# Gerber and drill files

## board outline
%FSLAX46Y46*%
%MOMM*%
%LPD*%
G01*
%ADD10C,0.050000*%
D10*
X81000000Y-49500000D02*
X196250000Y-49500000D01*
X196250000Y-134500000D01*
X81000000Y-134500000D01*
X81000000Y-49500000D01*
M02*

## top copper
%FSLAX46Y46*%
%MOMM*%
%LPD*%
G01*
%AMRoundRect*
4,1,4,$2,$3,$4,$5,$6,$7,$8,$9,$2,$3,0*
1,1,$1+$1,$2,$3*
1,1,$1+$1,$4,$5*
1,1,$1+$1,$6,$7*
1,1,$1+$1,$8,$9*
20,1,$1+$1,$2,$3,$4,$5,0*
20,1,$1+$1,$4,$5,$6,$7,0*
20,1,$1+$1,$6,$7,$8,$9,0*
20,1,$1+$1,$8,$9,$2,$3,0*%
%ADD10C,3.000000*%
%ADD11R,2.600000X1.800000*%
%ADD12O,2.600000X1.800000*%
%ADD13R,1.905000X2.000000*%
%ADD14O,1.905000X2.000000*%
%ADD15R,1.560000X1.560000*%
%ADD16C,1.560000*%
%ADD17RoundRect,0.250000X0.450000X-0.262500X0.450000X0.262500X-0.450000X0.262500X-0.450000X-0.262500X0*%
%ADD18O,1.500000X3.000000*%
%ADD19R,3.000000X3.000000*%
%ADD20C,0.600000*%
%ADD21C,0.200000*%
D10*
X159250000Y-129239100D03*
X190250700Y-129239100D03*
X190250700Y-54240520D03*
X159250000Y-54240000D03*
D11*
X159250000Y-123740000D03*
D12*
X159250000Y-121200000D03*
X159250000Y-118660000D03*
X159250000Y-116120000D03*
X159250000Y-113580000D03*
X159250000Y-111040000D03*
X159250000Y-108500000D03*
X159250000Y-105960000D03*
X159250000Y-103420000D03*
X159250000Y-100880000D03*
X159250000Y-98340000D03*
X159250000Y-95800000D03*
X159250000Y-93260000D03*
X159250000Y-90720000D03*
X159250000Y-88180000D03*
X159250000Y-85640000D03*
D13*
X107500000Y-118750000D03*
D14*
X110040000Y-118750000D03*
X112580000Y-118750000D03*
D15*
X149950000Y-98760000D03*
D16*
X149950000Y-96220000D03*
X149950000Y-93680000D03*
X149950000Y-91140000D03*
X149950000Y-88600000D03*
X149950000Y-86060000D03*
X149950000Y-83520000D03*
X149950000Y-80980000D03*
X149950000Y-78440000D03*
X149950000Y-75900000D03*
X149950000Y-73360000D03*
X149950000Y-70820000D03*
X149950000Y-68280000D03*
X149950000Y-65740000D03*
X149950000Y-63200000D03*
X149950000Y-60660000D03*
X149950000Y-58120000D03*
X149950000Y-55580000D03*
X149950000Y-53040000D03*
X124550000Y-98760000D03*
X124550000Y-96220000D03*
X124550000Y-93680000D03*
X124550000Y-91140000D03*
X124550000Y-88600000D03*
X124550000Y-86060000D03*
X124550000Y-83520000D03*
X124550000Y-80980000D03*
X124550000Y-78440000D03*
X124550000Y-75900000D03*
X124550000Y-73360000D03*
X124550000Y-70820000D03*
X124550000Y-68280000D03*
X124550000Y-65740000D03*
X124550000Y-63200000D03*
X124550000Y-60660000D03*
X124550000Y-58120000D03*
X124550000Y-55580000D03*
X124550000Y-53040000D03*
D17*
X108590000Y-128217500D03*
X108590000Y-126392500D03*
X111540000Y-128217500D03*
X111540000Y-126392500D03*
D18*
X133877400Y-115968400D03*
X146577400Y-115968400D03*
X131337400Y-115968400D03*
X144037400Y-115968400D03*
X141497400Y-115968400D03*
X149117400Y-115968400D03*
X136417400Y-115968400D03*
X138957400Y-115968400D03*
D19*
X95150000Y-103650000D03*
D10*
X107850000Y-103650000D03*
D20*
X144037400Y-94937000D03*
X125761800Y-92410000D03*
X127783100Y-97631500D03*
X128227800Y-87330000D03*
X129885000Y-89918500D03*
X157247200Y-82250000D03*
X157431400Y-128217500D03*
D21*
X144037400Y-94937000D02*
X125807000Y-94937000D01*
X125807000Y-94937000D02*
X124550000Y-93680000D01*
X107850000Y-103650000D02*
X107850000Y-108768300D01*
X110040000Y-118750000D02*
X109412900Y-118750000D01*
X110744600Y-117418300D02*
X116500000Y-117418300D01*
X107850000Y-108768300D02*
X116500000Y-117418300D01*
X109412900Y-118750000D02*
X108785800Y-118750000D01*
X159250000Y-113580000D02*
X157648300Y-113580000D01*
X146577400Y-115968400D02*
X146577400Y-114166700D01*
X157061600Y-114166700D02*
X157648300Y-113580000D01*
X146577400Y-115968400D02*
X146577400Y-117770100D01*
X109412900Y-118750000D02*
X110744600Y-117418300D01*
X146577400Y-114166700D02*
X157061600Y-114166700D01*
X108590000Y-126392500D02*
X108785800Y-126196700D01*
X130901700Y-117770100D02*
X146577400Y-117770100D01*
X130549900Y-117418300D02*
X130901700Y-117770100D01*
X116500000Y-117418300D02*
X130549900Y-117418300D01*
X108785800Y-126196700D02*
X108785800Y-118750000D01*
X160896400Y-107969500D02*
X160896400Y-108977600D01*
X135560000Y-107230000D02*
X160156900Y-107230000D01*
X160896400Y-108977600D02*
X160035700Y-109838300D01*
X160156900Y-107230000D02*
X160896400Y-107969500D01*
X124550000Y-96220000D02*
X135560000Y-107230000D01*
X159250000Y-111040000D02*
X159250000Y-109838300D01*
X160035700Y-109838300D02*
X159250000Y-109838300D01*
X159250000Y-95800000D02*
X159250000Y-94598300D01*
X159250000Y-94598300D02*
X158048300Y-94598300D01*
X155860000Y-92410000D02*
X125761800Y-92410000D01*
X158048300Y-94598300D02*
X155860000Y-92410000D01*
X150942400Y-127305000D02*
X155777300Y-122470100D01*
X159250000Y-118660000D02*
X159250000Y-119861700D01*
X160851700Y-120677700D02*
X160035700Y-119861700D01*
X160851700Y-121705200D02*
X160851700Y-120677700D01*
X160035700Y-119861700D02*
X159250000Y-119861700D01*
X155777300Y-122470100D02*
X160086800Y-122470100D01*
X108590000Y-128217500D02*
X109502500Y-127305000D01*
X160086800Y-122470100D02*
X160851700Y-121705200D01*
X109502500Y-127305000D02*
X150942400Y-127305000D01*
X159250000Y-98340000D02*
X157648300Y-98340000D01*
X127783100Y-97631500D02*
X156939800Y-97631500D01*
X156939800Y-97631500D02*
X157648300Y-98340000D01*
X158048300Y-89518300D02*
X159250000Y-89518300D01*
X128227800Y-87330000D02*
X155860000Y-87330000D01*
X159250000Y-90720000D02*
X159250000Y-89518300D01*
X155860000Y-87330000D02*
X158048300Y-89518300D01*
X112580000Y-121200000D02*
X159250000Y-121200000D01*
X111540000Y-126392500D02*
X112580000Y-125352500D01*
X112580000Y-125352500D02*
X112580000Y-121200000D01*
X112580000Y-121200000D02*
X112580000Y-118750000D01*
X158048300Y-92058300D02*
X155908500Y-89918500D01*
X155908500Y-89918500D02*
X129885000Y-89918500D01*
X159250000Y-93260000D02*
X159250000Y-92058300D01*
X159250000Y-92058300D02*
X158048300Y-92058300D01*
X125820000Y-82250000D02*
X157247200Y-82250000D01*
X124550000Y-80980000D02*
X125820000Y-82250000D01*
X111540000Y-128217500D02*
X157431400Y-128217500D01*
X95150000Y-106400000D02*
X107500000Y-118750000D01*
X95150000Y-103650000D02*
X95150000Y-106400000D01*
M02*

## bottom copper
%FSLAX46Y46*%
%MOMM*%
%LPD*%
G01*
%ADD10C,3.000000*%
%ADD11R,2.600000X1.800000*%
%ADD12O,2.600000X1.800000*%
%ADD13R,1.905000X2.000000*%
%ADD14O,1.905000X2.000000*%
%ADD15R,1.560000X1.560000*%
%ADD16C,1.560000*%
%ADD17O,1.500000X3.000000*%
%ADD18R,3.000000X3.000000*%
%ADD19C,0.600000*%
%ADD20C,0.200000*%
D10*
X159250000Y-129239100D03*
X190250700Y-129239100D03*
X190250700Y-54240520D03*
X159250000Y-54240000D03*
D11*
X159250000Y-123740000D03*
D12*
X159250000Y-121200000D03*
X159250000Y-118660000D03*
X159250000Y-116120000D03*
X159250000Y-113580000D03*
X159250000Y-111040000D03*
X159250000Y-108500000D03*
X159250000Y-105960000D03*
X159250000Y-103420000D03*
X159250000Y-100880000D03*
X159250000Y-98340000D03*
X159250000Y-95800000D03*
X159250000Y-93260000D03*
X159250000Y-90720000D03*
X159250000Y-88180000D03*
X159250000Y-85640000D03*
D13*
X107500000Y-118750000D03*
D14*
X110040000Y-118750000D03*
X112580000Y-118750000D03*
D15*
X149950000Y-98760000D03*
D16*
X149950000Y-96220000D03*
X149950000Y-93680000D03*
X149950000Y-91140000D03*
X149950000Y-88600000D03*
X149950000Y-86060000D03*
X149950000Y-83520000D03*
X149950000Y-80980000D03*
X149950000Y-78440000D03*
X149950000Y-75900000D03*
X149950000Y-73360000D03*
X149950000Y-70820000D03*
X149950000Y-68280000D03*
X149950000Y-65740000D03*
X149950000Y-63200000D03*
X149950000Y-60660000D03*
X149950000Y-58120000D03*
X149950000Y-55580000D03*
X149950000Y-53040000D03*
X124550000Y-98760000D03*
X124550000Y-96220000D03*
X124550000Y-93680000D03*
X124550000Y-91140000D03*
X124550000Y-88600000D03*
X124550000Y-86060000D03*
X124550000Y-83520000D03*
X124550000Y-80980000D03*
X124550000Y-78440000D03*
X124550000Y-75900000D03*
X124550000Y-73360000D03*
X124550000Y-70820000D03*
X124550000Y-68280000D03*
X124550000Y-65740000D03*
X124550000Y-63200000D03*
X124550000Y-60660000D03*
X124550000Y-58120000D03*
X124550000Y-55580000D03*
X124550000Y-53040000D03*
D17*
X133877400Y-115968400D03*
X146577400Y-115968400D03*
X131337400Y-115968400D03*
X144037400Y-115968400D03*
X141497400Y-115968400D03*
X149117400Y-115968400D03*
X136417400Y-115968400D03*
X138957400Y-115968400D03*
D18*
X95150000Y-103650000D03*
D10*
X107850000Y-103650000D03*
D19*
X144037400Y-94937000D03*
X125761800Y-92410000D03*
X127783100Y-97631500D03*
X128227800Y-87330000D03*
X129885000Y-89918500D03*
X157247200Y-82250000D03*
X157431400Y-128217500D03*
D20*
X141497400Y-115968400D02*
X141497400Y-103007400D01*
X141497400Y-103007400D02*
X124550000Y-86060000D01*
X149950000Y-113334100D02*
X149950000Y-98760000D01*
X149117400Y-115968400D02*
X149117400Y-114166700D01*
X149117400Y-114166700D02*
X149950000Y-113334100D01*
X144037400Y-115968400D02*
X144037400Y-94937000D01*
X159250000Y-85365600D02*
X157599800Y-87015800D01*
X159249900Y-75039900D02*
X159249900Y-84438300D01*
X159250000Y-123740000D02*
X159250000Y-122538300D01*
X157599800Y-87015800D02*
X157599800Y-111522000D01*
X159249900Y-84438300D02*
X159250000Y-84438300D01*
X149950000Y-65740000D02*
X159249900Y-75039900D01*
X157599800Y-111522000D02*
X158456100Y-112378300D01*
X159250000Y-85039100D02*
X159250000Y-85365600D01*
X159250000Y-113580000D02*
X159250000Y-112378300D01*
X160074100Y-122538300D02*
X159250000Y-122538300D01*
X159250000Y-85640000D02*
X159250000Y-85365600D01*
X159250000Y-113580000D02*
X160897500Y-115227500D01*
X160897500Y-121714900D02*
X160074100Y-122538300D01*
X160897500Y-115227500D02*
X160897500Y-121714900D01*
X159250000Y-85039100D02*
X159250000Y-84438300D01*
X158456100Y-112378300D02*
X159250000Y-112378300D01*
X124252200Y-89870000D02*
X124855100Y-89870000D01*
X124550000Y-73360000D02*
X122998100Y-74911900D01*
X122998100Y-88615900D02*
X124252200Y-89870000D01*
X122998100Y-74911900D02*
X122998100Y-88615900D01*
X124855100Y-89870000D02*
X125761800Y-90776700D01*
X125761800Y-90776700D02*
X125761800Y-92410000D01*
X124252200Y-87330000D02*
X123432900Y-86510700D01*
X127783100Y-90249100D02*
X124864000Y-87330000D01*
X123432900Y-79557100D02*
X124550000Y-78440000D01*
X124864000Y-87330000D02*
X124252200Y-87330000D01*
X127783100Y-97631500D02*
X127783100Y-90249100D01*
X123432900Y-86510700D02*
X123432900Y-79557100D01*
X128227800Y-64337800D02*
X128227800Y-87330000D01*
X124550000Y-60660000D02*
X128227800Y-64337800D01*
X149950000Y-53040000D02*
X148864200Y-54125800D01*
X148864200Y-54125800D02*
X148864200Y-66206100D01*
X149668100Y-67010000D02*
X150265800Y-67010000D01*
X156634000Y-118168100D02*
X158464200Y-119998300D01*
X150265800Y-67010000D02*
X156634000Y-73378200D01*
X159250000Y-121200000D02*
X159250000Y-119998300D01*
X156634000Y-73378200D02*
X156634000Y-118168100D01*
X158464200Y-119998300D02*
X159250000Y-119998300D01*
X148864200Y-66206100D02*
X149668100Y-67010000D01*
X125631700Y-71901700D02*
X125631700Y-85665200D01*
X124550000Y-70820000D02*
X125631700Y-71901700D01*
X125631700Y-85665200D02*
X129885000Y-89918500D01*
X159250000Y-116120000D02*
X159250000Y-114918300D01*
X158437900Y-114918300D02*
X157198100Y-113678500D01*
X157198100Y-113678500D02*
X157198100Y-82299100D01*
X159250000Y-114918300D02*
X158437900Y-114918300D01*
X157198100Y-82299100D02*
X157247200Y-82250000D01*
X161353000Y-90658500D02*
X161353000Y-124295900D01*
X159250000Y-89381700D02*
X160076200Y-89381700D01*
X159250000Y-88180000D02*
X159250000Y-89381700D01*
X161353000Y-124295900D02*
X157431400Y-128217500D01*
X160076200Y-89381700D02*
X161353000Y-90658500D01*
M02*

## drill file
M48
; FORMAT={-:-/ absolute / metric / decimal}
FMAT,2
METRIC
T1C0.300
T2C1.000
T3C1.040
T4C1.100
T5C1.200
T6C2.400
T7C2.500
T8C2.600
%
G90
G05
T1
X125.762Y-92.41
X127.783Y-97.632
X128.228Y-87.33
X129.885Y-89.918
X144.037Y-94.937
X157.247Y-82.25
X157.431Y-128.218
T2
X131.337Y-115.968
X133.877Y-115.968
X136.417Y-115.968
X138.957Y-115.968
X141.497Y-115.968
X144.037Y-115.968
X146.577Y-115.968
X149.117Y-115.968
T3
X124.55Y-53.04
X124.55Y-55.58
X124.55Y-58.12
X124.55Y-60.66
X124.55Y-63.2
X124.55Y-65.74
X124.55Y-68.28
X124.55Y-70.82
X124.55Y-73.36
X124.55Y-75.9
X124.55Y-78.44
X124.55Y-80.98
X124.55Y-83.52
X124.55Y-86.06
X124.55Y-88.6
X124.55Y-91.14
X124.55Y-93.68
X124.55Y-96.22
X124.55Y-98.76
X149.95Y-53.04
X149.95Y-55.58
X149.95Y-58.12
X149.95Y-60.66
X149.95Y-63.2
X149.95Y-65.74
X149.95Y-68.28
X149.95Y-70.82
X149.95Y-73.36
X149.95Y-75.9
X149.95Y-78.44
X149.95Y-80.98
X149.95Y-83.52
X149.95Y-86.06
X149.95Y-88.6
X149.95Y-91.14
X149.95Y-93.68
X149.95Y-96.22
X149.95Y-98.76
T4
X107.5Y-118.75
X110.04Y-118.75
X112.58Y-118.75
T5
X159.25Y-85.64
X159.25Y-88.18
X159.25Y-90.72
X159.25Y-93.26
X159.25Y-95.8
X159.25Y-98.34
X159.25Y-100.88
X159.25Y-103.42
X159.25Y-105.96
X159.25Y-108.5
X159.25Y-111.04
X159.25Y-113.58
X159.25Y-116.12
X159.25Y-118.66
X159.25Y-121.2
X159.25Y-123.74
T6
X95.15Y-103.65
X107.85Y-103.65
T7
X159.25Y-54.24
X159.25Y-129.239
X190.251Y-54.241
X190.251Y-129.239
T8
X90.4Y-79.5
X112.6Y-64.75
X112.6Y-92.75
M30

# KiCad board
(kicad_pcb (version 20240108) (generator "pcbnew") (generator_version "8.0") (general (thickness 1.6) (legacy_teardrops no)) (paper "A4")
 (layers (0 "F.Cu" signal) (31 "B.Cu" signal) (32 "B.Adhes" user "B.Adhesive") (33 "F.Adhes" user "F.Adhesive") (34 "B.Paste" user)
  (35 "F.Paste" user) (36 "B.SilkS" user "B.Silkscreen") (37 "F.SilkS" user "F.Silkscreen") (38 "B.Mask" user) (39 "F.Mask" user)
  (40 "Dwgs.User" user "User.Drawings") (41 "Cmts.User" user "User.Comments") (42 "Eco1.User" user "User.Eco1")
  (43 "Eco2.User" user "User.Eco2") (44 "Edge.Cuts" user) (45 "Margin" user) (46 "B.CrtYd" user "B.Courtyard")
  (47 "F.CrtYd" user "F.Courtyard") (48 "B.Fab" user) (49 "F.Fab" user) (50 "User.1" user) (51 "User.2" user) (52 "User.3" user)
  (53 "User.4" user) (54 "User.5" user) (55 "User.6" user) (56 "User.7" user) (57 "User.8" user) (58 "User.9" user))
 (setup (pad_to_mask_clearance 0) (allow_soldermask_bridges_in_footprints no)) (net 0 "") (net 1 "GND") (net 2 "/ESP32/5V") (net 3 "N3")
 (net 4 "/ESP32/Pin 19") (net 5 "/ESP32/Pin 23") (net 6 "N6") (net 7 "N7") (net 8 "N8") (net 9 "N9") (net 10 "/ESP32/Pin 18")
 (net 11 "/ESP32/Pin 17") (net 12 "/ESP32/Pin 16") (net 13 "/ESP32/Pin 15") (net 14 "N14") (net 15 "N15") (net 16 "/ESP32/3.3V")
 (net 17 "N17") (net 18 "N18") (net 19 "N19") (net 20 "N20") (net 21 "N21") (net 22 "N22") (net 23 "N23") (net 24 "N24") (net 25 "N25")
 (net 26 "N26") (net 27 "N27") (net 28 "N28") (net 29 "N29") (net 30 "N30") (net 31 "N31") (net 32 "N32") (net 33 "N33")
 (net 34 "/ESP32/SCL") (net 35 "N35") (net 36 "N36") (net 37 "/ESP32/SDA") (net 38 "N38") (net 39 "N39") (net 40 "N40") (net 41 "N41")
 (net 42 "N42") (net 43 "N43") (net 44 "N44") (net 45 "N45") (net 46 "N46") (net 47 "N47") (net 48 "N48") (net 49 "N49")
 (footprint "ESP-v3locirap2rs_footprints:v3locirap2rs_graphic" (layer "F.Cu") (at 90 122.5)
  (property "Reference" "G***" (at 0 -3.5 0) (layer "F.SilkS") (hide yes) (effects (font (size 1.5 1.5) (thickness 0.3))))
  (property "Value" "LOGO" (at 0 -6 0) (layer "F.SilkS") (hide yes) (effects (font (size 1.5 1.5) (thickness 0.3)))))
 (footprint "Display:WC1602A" (layer "F.Cu") (at 159.25 123.74 90)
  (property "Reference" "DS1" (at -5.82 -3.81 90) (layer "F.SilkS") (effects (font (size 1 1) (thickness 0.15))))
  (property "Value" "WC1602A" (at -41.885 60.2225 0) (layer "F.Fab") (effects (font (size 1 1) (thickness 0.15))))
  (pad "" thru_hole circle (at -5.4991 0 90) (size 3 3) (drill 2.5) (layers "*.Cu" "*.Mask") (remove_unused_layers no))
  (pad "" thru_hole circle (at -5.4991 31.0007 90) (size 3 3) (drill 2.5) (layers "*.Cu" "*.Mask") (remove_unused_layers no))
  (pad "" thru_hole circle (at 69.49948 31.0007 90) (size 3 3) (drill 2.5) (layers "*.Cu" "*.Mask") (remove_unused_layers no))
  (pad "" thru_hole circle (at 69.5 0 90) (size 3 3) (drill 2.5) (layers "*.Cu" "*.Mask") (remove_unused_layers no))
  (pad "1" thru_hole rect (at 0 0 90) (size 1.8 2.6) (drill 1.2) (layers "*.Cu" "*.Mask") (remove_unused_layers no) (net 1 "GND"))
  (pad "2" thru_hole oval (at 2.54 0 90) (size 1.8 2.6) (drill 1.2) (layers "*.Cu" "*.Mask") (remove_unused_layers no) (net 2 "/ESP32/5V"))
  (pad "3" thru_hole oval (at 5.08 0 90) (size 1.8 2.6) (drill 1.2) (layers "*.Cu" "*.Mask") (remove_unused_layers no) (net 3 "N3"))
  (pad "4" thru_hole oval (at 7.62 0 90) (size 1.8 2.6) (drill 1.2) (layers "*.Cu" "*.Mask") (remove_unused_layers no)
   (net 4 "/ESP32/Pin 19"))
  (pad "5" thru_hole oval (at 10.16 0 90) (size 1.8 2.6) (drill 1.2) (layers "*.Cu" "*.Mask") (remove_unused_layers no) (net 1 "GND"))
  (pad "6" thru_hole oval (at 12.7 0 90) (size 1.8 2.6) (drill 1.2) (layers "*.Cu" "*.Mask") (remove_unused_layers no)
   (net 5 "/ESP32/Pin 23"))
  (pad "7" thru_hole oval (at 15.24 0 90) (size 1.8 2.6) (drill 1.2) (layers "*.Cu" "*.Mask") (remove_unused_layers no) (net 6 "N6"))
  (pad "8" thru_hole oval (at 17.78 0 90) (size 1.8 2.6) (drill 1.2) (layers "*.Cu" "*.Mask") (remove_unused_layers no) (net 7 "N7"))
  (pad "9" thru_hole oval (at 20.32 0 90) (size 1.8 2.6) (drill 1.2) (layers "*.Cu" "*.Mask") (remove_unused_layers no) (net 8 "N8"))
  (pad "10" thru_hole oval (at 22.86 0 90) (size 1.8 2.6) (drill 1.2) (layers "*.Cu" "*.Mask") (remove_unused_layers no) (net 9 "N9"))
  (pad "11" thru_hole oval (at 25.4 0 90) (size 1.8 2.6) (drill 1.2) (layers "*.Cu" "*.Mask") (remove_unused_layers no)
   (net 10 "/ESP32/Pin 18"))
  (pad "12" thru_hole oval (at 27.94 0 90) (size 1.8 2.6) (drill 1.2) (layers "*.Cu" "*.Mask") (remove_unused_layers no)
   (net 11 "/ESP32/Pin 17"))
  (pad "13" thru_hole oval (at 30.48 0 90) (size 1.8 2.6) (drill 1.2) (layers "*.Cu" "*.Mask") (remove_unused_layers no)
   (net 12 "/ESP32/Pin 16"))
  (pad "14" thru_hole oval (at 33.02 0 90) (size 1.8 2.6) (drill 1.2) (layers "*.Cu" "*.Mask") (remove_unused_layers no)
   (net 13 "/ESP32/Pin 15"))
  (pad "15" thru_hole oval (at 35.56 0 90) (size 1.8 2.6) (drill 1.2) (layers "*.Cu" "*.Mask") (remove_unused_layers no) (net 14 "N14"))
  (pad "16" thru_hole oval (at 38.1 0 90) (size 1.8 2.6) (drill 1.2) (layers "*.Cu" "*.Mask") (remove_unused_layers no) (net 1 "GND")))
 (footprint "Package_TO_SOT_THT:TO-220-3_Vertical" (layer "F.Cu") (at 107.5 118.75)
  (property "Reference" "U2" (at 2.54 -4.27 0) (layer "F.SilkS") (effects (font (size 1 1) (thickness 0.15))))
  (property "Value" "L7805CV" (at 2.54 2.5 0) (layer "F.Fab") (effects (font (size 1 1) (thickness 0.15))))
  (pad "1" thru_hole rect (at 0 0) (size 1.905 2) (drill 1.1) (layers "*.Cu" "*.Mask") (remove_unused_layers no) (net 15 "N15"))
  (pad "2" thru_hole oval (at 2.54 0) (size 1.905 2) (drill 1.1) (layers "*.Cu" "*.Mask") (remove_unused_layers no) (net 1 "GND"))
  (pad "3" thru_hole oval (at 5.08 0) (size 1.905 2) (drill 1.1) (layers "*.Cu" "*.Mask") (remove_unused_layers no) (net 2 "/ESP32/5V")))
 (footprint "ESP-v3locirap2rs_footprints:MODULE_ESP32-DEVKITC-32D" (layer "F.Cu") (at 137.25 79 180)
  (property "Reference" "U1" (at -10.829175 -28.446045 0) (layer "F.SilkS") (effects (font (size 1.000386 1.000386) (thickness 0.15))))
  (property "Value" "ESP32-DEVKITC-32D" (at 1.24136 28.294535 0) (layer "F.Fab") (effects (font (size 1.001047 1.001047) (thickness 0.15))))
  (pad "J2-1" thru_hole rect (at -12.7 -19.76 180) (size 1.56 1.56) (drill 1.04) (layers "*.Cu" "*.Mask") (remove_unused_layers no)
   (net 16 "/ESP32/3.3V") (solder_mask_margin 0.102))
  (pad "J2-2" thru_hole circle (at -12.7 -17.22 180) (size 1.56 1.56) (drill 1.04) (layers "*.Cu" "*.Mask") (remove_unused_layers no)
   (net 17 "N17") (solder_mask_margin 0.102))
  (pad "J2-3" thru_hole circle (at -12.7 -14.68 180) (size 1.56 1.56) (drill 1.04) (layers "*.Cu" "*.Mask") (remove_unused_layers no)
   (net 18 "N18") (solder_mask_margin 0.102))
  (pad "J2-4" thru_hole circle (at -12.7 -12.14 180) (size 1.56 1.56) (drill 1.04) (layers "*.Cu" "*.Mask") (remove_unused_layers no)
   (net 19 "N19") (solder_mask_margin 0.102))
  (pad "J2-5" thru_hole circle (at -12.7 -9.6 180) (size 1.56 1.56) (drill 1.04) (layers "*.Cu" "*.Mask") (remove_unused_layers no)
   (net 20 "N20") (solder_mask_margin 0.102))
  (pad "J2-6" thru_hole circle (at -12.7 -7.06 180) (size 1.56 1.56) (drill 1.04) (layers "*.Cu" "*.Mask") (remove_unused_layers no)
   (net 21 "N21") (solder_mask_margin 0.102))
  (pad "J2-7" thru_hole circle (at -12.7 -4.52 180) (size 1.56 1.56) (drill 1.04) (layers "*.Cu" "*.Mask") (remove_unused_layers no)
   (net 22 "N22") (solder_mask_margin 0.102))
  (pad "J2-8" thru_hole circle (at -12.7 -1.98 180) (size 1.56 1.56) (drill 1.04) (layers "*.Cu" "*.Mask") (remove_unused_layers no)
   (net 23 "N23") (solder_mask_margin 0.102))
  (pad "J2-9" thru_hole circle (at -12.7 0.56 180) (size 1.56 1.56) (drill 1.04) (layers "*.Cu" "*.Mask") (remove_unused_layers no)
   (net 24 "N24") (solder_mask_margin 0.102))
  (pad "J2-10" thru_hole circle (at -12.7 3.1 180) (size 1.56 1.56) (drill 1.04) (layers "*.Cu" "*.Mask") (remove_unused_layers no)
   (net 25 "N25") (solder_mask_margin 0.102))
  (pad "J2-11" thru_hole circle (at -12.7 5.64 180) (size 1.56 1.56) (drill 1.04) (layers "*.Cu" "*.Mask") (remove_unused_layers no)
   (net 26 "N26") (solder_mask_margin 0.102))
  (pad "J2-12" thru_hole circle (at -12.7 8.18 180) (size 1.56 1.56) (drill 1.04) (layers "*.Cu" "*.Mask") (remove_unused_layers no)
   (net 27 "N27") (solder_mask_margin 0.102))
  (pad "J2-13" thru_hole circle (at -12.7 10.72 180) (size 1.56 1.56) (drill 1.04) (layers "*.Cu" "*.Mask") (remove_unused_layers no)
   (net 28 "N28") (solder_mask_margin 0.102))
  (pad "J2-14" thru_hole circle (at -12.7 13.26 180) (size 1.56 1.56) (drill 1.04) (layers "*.Cu" "*.Mask") (remove_unused_layers no)
   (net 1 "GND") (solder_mask_margin 0.102))
  (pad "J2-15" thru_hole circle (at -12.7 15.8 180) (size 1.56 1.56) (drill 1.04) (layers "*.Cu" "*.Mask") (remove_unused_layers no)
   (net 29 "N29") (solder_mask_margin 0.102))
  (pad "J2-16" thru_hole circle (at -12.7 18.34 180) (size 1.56 1.56) (drill 1.04) (layers "*.Cu" "*.Mask") (remove_unused_layers no)
   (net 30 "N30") (solder_mask_margin 0.102))
  (pad "J2-17" thru_hole circle (at -12.7 20.88 180) (size 1.56 1.56) (drill 1.04) (layers "*.Cu" "*.Mask") (remove_unused_layers no)
   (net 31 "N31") (solder_mask_margin 0.102))
  (pad "J2-18" thru_hole circle (at -12.7 23.42 180) (size 1.56 1.56) (drill 1.04) (layers "*.Cu" "*.Mask") (remove_unused_layers no)
   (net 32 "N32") (solder_mask_margin 0.102))
  (pad "J2-19" thru_hole circle (at -12.7 25.96 180) (size 1.56 1.56) (drill 1.04) (layers "*.Cu" "*.Mask") (remove_unused_layers no)
   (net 2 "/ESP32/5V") (solder_mask_margin 0.102))
  (pad "J3-1" thru_hole circle (at 12.7 -19.76 180) (size 1.56 1.56) (drill 1.04) (layers "*.Cu" "*.Mask") (remove_unused_layers no)
   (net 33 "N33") (solder_mask_margin 0.102))
  (pad "J3-2" thru_hole circle (at 12.7 -17.22 180) (size 1.56 1.56) (drill 1.04) (layers "*.Cu" "*.Mask") (remove_unused_layers no)
   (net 5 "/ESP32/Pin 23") (solder_mask_margin 0.102))
  (pad "J3-3" thru_hole circle (at 12.7 -14.68 180) (size 1.56 1.56) (drill 1.04) (layers "*.Cu" "*.Mask") (remove_unused_layers no)
   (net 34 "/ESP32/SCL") (solder_mask_margin 0.102))
  (pad "J3-4" thru_hole circle (at 12.7 -12.14 180) (size 1.56 1.56) (drill 1.04) (layers "*.Cu" "*.Mask") (remove_unused_layers no)
   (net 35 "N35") (solder_mask_margin 0.102))
  (pad "J3-5" thru_hole circle (at 12.7 -9.6 180) (size 1.56 1.56) (drill 1.04) (layers "*.Cu" "*.Mask") (remove_unused_layers no)
   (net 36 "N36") (solder_mask_margin 0.102))
  (pad "J3-6" thru_hole circle (at 12.7 -7.06 180) (size 1.56 1.56) (drill 1.04) (layers "*.Cu" "*.Mask") (remove_unused_layers no)
   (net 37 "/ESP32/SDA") (solder_mask_margin 0.102))
  (pad "J3-7" thru_hole circle (at 12.7 -4.52 180) (size 1.56 1.56) (drill 1.04) (layers "*.Cu" "*.Mask") (remove_unused_layers no)
   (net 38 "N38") (solder_mask_margin 0.102))
  (pad "J3-8" thru_hole circle (at 12.7 -1.98 180) (size 1.56 1.56) (drill 1.04) (layers "*.Cu" "*.Mask") (remove_unused_layers no)
   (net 4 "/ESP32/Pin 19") (solder_mask_margin 0.102))
  (pad "J3-9" thru_hole circle (at 12.7 0.56 180) (size 1.56 1.56) (drill 1.04) (layers "*.Cu" "*.Mask") (remove_unused_layers no)
   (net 10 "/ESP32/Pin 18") (solder_mask_margin 0.102))
  (pad "J3-10" thru_hole circle (at 12.7 3.1 180) (size 1.56 1.56) (drill 1.04) (layers "*.Cu" "*.Mask") (remove_unused_layers no)
   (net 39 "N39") (solder_mask_margin 0.102))
  (pad "J3-11" thru_hole circle (at 12.7 5.64 180) (size 1.56 1.56) (drill 1.04) (layers "*.Cu" "*.Mask") (remove_unused_layers no)
   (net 11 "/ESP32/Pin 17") (solder_mask_margin 0.102))
  (pad "J3-12" thru_hole circle (at 12.7 8.18 180) (size 1.56 1.56) (drill 1.04) (layers "*.Cu" "*.Mask") (remove_unused_layers no)
   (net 12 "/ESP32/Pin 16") (solder_mask_margin 0.102))
  (pad "J3-13" thru_hole circle (at 12.7 10.72 180) (size 1.56 1.56) (drill 1.04) (layers "*.Cu" "*.Mask") (remove_unused_layers no)
   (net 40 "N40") (solder_mask_margin 0.102))
  (pad "J3-14" thru_hole circle (at 12.7 13.26 180) (size 1.56 1.56) (drill 1.04) (layers "*.Cu" "*.Mask") (remove_unused_layers no)
   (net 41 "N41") (solder_mask_margin 0.102))
  (pad "J3-15" thru_hole circle (at 12.7 15.8 180) (size 1.56 1.56) (drill 1.04) (layers "*.Cu" "*.Mask") (remove_unused_layers no)
   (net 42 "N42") (solder_mask_margin 0.102))
  (pad "J3-16" thru_hole circle (at 12.7 18.34 180) (size 1.56 1.56) (drill 1.04) (layers "*.Cu" "*.Mask") (remove_unused_layers no)
   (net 13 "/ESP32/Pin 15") (solder_mask_margin 0.102))
  (pad "J3-17" thru_hole circle (at 12.7 20.88 180) (size 1.56 1.56) (drill 1.04) (layers "*.Cu" "*.Mask") (remove_unused_layers no)
   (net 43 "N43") (solder_mask_margin 0.102))
  (pad "J3-18" thru_hole circle (at 12.7 23.42 180) (size 1.56 1.56) (drill 1.04) (layers "*.Cu" "*.Mask") (remove_unused_layers no)
   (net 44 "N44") (solder_mask_margin 0.102))
  (pad "J3-19" thru_hole circle (at 12.7 25.96 180) (size 1.56 1.56) (drill 1.04) (layers "*.Cu" "*.Mask") (remove_unused_layers no)
   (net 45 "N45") (solder_mask_margin 0.102)))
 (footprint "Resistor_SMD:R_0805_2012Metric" (layer "F.Cu") (at 108.59 127.305 90)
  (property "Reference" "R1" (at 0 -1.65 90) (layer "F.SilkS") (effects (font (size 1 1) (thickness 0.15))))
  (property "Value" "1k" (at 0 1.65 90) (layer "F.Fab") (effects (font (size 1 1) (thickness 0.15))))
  (pad "1" smd roundrect (at -0.9125 0 90) (size 1.025 1.4) (layers "F.Cu" "F.Paste" "F.Mask") (roundrect_rratio 0.243902) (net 3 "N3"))
  (pad "2" smd roundrect (at 0.9125 0 90) (size 1.025 1.4) (layers "F.Cu" "F.Paste" "F.Mask") (roundrect_rratio 0.243902) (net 1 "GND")))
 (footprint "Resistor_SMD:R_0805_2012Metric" (layer "F.Cu") (at 111.54 127.305 90)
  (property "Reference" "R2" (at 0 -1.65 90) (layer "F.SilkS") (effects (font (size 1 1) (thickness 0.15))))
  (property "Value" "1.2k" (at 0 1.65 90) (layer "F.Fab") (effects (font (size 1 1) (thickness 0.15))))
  (pad "1" smd roundrect (at -0.9125 0 90) (size 1.025 1.4) (layers "F.Cu" "F.Paste" "F.Mask") (roundrect_rratio 0.243902) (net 14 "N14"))
  (pad "2" smd roundrect (at 0.9125 0 90) (size 1.025 1.4) (layers "F.Cu" "F.Paste" "F.Mask") (roundrect_rratio 0.243902)
   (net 2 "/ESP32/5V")))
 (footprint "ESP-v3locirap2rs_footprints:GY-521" (layer "F.Cu") (at 129.2734 114.1984 -90)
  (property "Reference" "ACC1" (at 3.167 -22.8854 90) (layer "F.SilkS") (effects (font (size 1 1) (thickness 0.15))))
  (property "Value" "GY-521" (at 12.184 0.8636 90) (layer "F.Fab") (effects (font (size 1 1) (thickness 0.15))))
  (pad "AD0" thru_hole oval (at 1.77 -4.604 270) (size 3 1.5) (drill 1) (layers "*.Cu" "*.Mask") (remove_unused_layers no) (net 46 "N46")
   (solder_mask_margin 0.102))
  (pad "GND" thru_hole oval (at 1.77 -17.304 270) (size 3 1.5) (drill 1) (layers "*.Cu" "*.Mask") (remove_unused_layers no) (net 1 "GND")
   (solder_mask_margin 0.102))
  (pad "INT" thru_hole oval (at 1.77 -2.064 270) (size 3 1.5) (drill 1) (layers "*.Cu" "*.Mask") (remove_unused_layers no) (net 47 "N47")
   (solder_mask_margin 0.102))
  (pad "SCL" thru_hole oval (at 1.77 -14.764 270) (size 3 1.5) (drill 1) (layers "*.Cu" "*.Mask") (remove_unused_layers no)
   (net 34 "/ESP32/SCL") (solder_mask_margin 0.102))
  (pad "SDA" thru_hole oval (at 1.77 -12.224 270) (size 3 1.5) (drill 1) (layers "*.Cu" "*.Mask") (remove_unused_layers no)
   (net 37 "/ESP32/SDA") (solder_mask_margin 0.102))
  (pad "VCC" thru_hole oval (at 1.77 -19.844 270) (size 3 1.5) (drill 1) (layers "*.Cu" "*.Mask") (remove_unused_layers no)
   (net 16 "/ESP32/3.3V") (solder_mask_margin 0.102))
  (pad "XCL" thru_hole oval (at 1.77 -7.144 270) (size 3 1.5) (drill 1) (layers "*.Cu" "*.Mask") (remove_unused_layers no) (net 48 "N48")
   (solder_mask_margin 0.102))
  (pad "XDA" thru_hole oval (at 1.77 -9.684 270) (size 3 1.5) (drill 1) (layers "*.Cu" "*.Mask") (remove_unused_layers no) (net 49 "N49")
   (solder_mask_margin 0.102)))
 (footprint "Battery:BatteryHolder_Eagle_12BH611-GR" (layer "F.Cu") (at 95.15 103.65 -90)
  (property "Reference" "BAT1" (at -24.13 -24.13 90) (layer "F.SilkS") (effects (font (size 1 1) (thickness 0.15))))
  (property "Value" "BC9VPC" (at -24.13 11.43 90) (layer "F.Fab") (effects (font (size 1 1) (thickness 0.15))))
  (pad "" np_thru_hole circle (at -38.9 -17.45 270) (size 2.6 2.6) (drill 2.6) (layers "*.Cu" "*.Mask"))
  (pad "" np_thru_hole circle (at -24.15 4.75 270) (size 2.6 2.6) (drill 2.6) (layers "*.Cu" "*.Mask"))
  (pad "" np_thru_hole circle (at -10.9 -17.45 270) (size 2.6 2.6) (drill 2.6) (layers "*.Cu" "*.Mask"))
  (pad "1" thru_hole rect (at 0 0 270) (size 3 3) (drill 2.4) (layers "*.Cu" "*.Mask") (remove_unused_layers no) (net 15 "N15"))
  (pad "2" thru_hole circle (at 0 -12.7 270) (size 3 3) (drill 2.4) (layers "*.Cu" "*.Mask") (remove_unused_layers no) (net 1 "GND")))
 (gr_rect (start 81 49.5) (end 196.25 134.5) (stroke (width 0.05) (type default)) (fill none) (layer "Edge.Cuts"))
 (segment (start 141.4974 115.9684) (end 141.4974 103.0074) (width 0.2) (layer "B.Cu") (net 37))
 (segment (start 141.4974 103.0074) (end 124.55 86.06) (width 0.2) (layer "B.Cu") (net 37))
 (segment (start 149.95 113.3341) (end 149.95 98.76) (width 0.2) (layer "B.Cu") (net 16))
 (segment (start 149.1174 115.9684) (end 149.1174 114.1667) (width 0.2) (layer "B.Cu") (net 16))
 (segment (start 149.1174 114.1667) (end 149.95 113.3341) (width 0.2) (layer "B.Cu") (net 16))
 (segment (start 144.0374 94.937) (end 125.807 94.937) (width 0.2) (layer "F.Cu") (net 34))
 (segment (start 125.807 94.937) (end 124.55 93.68) (width 0.2) (layer "F.Cu") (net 34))
 (via (at 144.0374 94.937) (size 0.6) (drill 0.3) (layers "F.Cu" "B.Cu") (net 34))
 (segment (start 144.0374 115.9684) (end 144.0374 94.937) (width 0.2) (layer "B.Cu") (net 34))
 (segment (start 107.85 103.65) (end 107.85 108.7683) (width 0.2) (layer "F.Cu") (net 1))
 (segment (start 110.04 118.75) (end 109.4129 118.75) (width 0.2) (layer "F.Cu") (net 1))
 (segment (start 110.7446 117.4183) (end 116.5 117.4183) (width 0.2) (layer "F.Cu") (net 1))
 (segment (start 107.85 108.7683) (end 116.5 117.4183) (width 0.2) (layer "F.Cu") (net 1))
 (segment (start 109.4129 118.75) (end 108.7858 118.75) (width 0.2) (layer "F.Cu") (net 1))
 (segment (start 159.25 113.58) (end 157.6483 113.58) (width 0.2) (layer "F.Cu") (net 1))
 (segment (start 146.5774 115.9684) (end 146.5774 114.1667) (width 0.2) (layer "F.Cu") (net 1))
 (segment (start 157.0616 114.1667) (end 157.6483 113.58) (width 0.2) (layer "F.Cu") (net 1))
 (segment (start 146.5774 115.9684) (end 146.5774 117.7701) (width 0.2) (layer "F.Cu") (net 1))
 (segment (start 109.4129 118.75) (end 110.7446 117.4183) (width 0.2) (layer "F.Cu") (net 1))
 (segment (start 146.5774 114.1667) (end 157.0616 114.1667) (width 0.2) (layer "F.Cu") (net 1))
 (segment (start 108.59 126.3925) (end 108.7858 126.1967) (width 0.2) (layer "F.Cu") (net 1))
 (segment (start 130.9017 117.7701) (end 146.5774 117.7701) (width 0.2) (layer "F.Cu") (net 1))
 (segment (start 130.5499 117.4183) (end 130.9017 117.7701) (width 0.2) (layer "F.Cu") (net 1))
 (segment (start 116.5 117.4183) (end 130.5499 117.4183) (width 0.2) (layer "F.Cu") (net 1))
 (segment (start 108.7858 126.1967) (end 108.7858 118.75) (width 0.2) (layer "F.Cu") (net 1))
 (segment (start 159.25 85.3656) (end 157.5998 87.0158) (width 0.2) (layer "B.Cu") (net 1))
 (segment (start 159.2499 75.0399) (end 159.2499 84.4383) (width 0.2) (layer "B.Cu") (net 1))
 (segment (start 159.25 123.74) (end 159.25 122.5383) (width 0.2) (layer "B.Cu") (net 1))
 (segment (start 157.5998 87.0158) (end 157.5998 111.522) (width 0.2) (layer "B.Cu") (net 1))
 (segment (start 159.2499 84.4383) (end 159.25 84.4383) (width 0.2) (layer "B.Cu") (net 1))
 (segment (start 149.95 65.74) (end 159.2499 75.0399) (width 0.2) (layer "B.Cu") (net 1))
 (segment (start 157.5998 111.522) (end 158.4561 112.3783) (width 0.2) (layer "B.Cu") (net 1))
 (segment (start 159.25 85.0391) (end 159.25 85.3656) (width 0.2) (layer "B.Cu") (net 1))
 (segment (start 159.25 113.58) (end 159.25 112.3783) (width 0.2) (layer "B.Cu") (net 1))
 (segment (start 160.0741 122.5383) (end 159.25 122.5383) (width 0.2) (layer "B.Cu") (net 1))
 (segment (start 159.25 85.64) (end 159.25 85.3656) (width 0.2) (layer "B.Cu") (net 1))
 (segment (start 159.25 113.58) (end 160.8975 115.2275) (width 0.2) (layer "B.Cu") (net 1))
 (segment (start 160.8975 121.7149) (end 160.0741 122.5383) (width 0.2) (layer "B.Cu") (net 1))
 (segment (start 160.8975 115.2275) (end 160.8975 121.7149) (width 0.2) (layer "B.Cu") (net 1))
 (segment (start 159.25 85.0391) (end 159.25 84.4383) (width 0.2) (layer "B.Cu") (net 1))
 (segment (start 158.4561 112.3783) (end 159.25 112.3783) (width 0.2) (layer "B.Cu") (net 1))
 (segment (start 160.8964 107.9695) (end 160.8964 108.9776) (width 0.2) (layer "F.Cu") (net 5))
 (segment (start 135.56 107.23) (end 160.1569 107.23) (width 0.2) (layer "F.Cu") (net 5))
 (segment (start 160.8964 108.9776) (end 160.0357 109.8383) (width 0.2) (layer "F.Cu") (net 5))
 (segment (start 160.1569 107.23) (end 160.8964 107.9695) (width 0.2) (layer "F.Cu") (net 5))
 (segment (start 124.55 96.22) (end 135.56 107.23) (width 0.2) (layer "F.Cu") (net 5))
 (segment (start 159.25 111.04) (end 159.25 109.8383) (width 0.2) (layer "F.Cu") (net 5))
 (segment (start 160.0357 109.8383) (end 159.25 109.8383) (width 0.2) (layer "F.Cu") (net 5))
 (segment (start 159.25 95.8) (end 159.25 94.5983) (width 0.2) (layer "F.Cu") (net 11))
 (segment (start 159.25 94.5983) (end 158.0483 94.5983) (width 0.2) (layer "F.Cu") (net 11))
 (segment (start 155.86 92.41) (end 125.7618 92.41) (width 0.2) (layer "F.Cu") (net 11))
 (segment (start 158.0483 94.5983) (end 155.86 92.41) (width 0.2) (layer "F.Cu") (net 11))
 (via (at 125.7618 92.41) (size 0.6) (drill 0.3) (layers "F.Cu" "B.Cu") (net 11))
 (segment (start 124.2522 89.87) (end 124.8551 89.87) (width 0.2) (layer "B.Cu") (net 11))
 (segment (start 124.55 73.36) (end 122.9981 74.9119) (width 0.2) (layer "B.Cu") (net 11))
 (segment (start 122.9981 88.6159) (end 124.2522 89.87) (width 0.2) (layer "B.Cu") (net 11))
 (segment (start 122.9981 74.9119) (end 122.9981 88.6159) (width 0.2) (layer "B.Cu") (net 11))
 (segment (start 124.8551 89.87) (end 125.7618 90.7767) (width 0.2) (layer "B.Cu") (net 11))
 (segment (start 125.7618 90.7767) (end 125.7618 92.41) (width 0.2) (layer "B.Cu") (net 11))
 (segment (start 150.9424 127.305) (end 155.7773 122.4701) (width 0.2) (layer "F.Cu") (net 3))
 (segment (start 159.25 118.66) (end 159.25 119.8617) (width 0.2) (layer "F.Cu") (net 3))
 (segment (start 160.8517 120.6777) (end 160.0357 119.8617) (width 0.2) (layer "F.Cu") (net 3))
 (segment (start 160.8517 121.7052) (end 160.8517 120.6777) (width 0.2) (layer "F.Cu") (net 3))
 (segment (start 160.0357 119.8617) (end 159.25 119.8617) (width 0.2) (layer "F.Cu") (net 3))
 (segment (start 155.7773 122.4701) (end 160.0868 122.4701) (width 0.2) (layer "F.Cu") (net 3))
 (segment (start 108.59 128.2175) (end 109.5025 127.305) (width 0.2) (layer "F.Cu") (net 3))
 (segment (start 160.0868 122.4701) (end 160.8517 121.7052) (width 0.2) (layer "F.Cu") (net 3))
 (segment (start 109.5025 127.305) (end 150.9424 127.305) (width 0.2) (layer "F.Cu") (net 3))
 (segment (start 159.25 98.34) (end 157.6483 98.34) (width 0.2) (layer "F.Cu") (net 10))
 (segment (start 127.7831 97.6315) (end 156.9398 97.6315) (width 0.2) (layer "F.Cu") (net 10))
 (segment (start 156.9398 97.6315) (end 157.6483 98.34) (width 0.2) (layer "F.Cu") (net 10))
 (via (at 127.7831 97.6315) (size 0.6) (drill 0.3) (layers "F.Cu" "B.Cu") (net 10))
 (segment (start 124.2522 87.33) (end 123.4329 86.5107) (width 0.2) (layer "B.Cu") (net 10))
 (segment (start 127.7831 90.2491) (end 124.864 87.33) (width 0.2) (layer "B.Cu") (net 10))
 (segment (start 123.4329 79.5571) (end 124.55 78.44) (width 0.2) (layer "B.Cu") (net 10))
 (segment (start 124.864 87.33) (end 124.2522 87.33) (width 0.2) (layer "B.Cu") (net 10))
 (segment (start 127.7831 97.6315) (end 127.7831 90.2491) (width 0.2) (layer "B.Cu") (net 10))
 (segment (start 123.4329 86.5107) (end 123.4329 79.5571) (width 0.2) (layer "B.Cu") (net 10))
 (segment (start 158.0483 89.5183) (end 159.25 89.5183) (width 0.2) (layer "F.Cu") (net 13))
 (segment (start 128.2278 87.33) (end 155.86 87.33) (width 0.2) (layer "F.Cu") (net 13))
 (segment (start 159.25 90.72) (end 159.25 89.5183) (width 0.2) (layer "F.Cu") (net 13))
 (segment (start 155.86 87.33) (end 158.0483 89.5183) (width 0.2) (layer "F.Cu") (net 13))
 (via (at 128.2278 87.33) (size 0.6) (drill 0.3) (layers "F.Cu" "B.Cu") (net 13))
 (segment (start 128.2278 64.3378) (end 128.2278 87.33) (width 0.2) (layer "B.Cu") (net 13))
 (segment (start 124.55 60.66) (end 128.2278 64.3378) (width 0.2) (layer "B.Cu") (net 13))
 (segment (start 112.58 121.2) (end 159.25 121.2) (width 0.2) (layer "F.Cu") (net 2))
 (segment (start 111.54 126.3925) (end 112.58 125.3525) (width 0.2) (layer "F.Cu") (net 2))
 (segment (start 112.58 125.3525) (end 112.58 121.2) (width 0.2) (layer "F.Cu") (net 2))
 (segment (start 112.58 121.2) (end 112.58 118.75) (width 0.2) (layer "F.Cu") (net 2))
 (segment (start 149.95 53.04) (end 148.8642 54.1258) (width 0.2) (layer "B.Cu") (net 2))
 (segment (start 148.8642 54.1258) (end 148.8642 66.2061) (width 0.2) (layer "B.Cu") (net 2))
 (segment (start 149.6681 67.01) (end 150.2658 67.01) (width 0.2) (layer "B.Cu") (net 2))
 (segment (start 156.634 118.1681) (end 158.4642 119.9983) (width 0.2) (layer "B.Cu") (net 2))
 (segment (start 150.2658 67.01) (end 156.634 73.3782) (width 0.2) (layer "B.Cu") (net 2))
 (segment (start 159.25 121.2) (end 159.25 119.9983) (width 0.2) (layer "B.Cu") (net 2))
 (segment (start 156.634 73.3782) (end 156.634 118.1681) (width 0.2) (layer "B.Cu") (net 2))
 (segment (start 158.4642 119.9983) (end 159.25 119.9983) (width 0.2) (layer "B.Cu") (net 2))
 (segment (start 148.8642 66.2061) (end 149.6681 67.01) (width 0.2) (layer "B.Cu") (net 2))
 (segment (start 158.0483 92.0583) (end 155.9085 89.9185) (width 0.2) (layer "F.Cu") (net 12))
 (segment (start 155.9085 89.9185) (end 129.885 89.9185) (width 0.2) (layer "F.Cu") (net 12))
 (segment (start 159.25 93.26) (end 159.25 92.0583) (width 0.2) (layer "F.Cu") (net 12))
 (segment (start 159.25 92.0583) (end 158.0483 92.0583) (width 0.2) (layer "F.Cu") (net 12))
 (via (at 129.885 89.9185) (size 0.6) (drill 0.3) (layers "F.Cu" "B.Cu") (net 12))
 (segment (start 125.6317 71.9017) (end 125.6317 85.6652) (width 0.2) (layer "B.Cu") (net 12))
 (segment (start 124.55 70.82) (end 125.6317 71.9017) (width 0.2) (layer "B.Cu") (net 12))
 (segment (start 125.6317 85.6652) (end 129.885 89.9185) (width 0.2) (layer "B.Cu") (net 12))
 (segment (start 125.82 82.25) (end 157.2472 82.25) (width 0.2) (layer "F.Cu") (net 4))
 (segment (start 124.55 80.98) (end 125.82 82.25) (width 0.2) (layer "F.Cu") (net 4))
 (via (at 157.2472 82.25) (size 0.6) (drill 0.3) (layers "F.Cu" "B.Cu") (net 4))
 (segment (start 159.25 116.12) (end 159.25 114.9183) (width 0.2) (layer "B.Cu") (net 4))
 (segment (start 158.4379 114.9183) (end 157.1981 113.6785) (width 0.2) (layer "B.Cu") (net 4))
 (segment (start 157.1981 113.6785) (end 157.1981 82.2991) (width 0.2) (layer "B.Cu") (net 4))
 (segment (start 159.25 114.9183) (end 158.4379 114.9183) (width 0.2) (layer "B.Cu") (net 4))
 (segment (start 157.1981 82.2991) (end 157.2472 82.25) (width 0.2) (layer "B.Cu") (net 4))
 (segment (start 111.54 128.2175) (end 157.4314 128.2175) (width 0.2) (layer "F.Cu") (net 14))
 (via (at 157.4314 128.2175) (size 0.6) (drill 0.3) (layers "F.Cu" "B.Cu") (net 14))
 (segment (start 161.353 90.6585) (end 161.353 124.2959) (width 0.2) (layer "B.Cu") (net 14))
 (segment (start 159.25 89.3817) (end 160.0762 89.3817) (width 0.2) (layer "B.Cu") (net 14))
 (segment (start 159.25 88.18) (end 159.25 89.3817) (width 0.2) (layer "B.Cu") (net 14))
 (segment (start 161.353 124.2959) (end 157.4314 128.2175) (width 0.2) (layer "B.Cu") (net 14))
 (segment (start 160.0762 89.3817) (end 161.353 90.6585) (width 0.2) (layer "B.Cu") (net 14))
 (segment (start 95.15 106.4) (end 107.5 118.75) (width 0.2) (layer "F.Cu") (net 15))
 (segment (start 95.15 103.65) (end 95.15 106.4) (width 0.2) (layer "F.Cu") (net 15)))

